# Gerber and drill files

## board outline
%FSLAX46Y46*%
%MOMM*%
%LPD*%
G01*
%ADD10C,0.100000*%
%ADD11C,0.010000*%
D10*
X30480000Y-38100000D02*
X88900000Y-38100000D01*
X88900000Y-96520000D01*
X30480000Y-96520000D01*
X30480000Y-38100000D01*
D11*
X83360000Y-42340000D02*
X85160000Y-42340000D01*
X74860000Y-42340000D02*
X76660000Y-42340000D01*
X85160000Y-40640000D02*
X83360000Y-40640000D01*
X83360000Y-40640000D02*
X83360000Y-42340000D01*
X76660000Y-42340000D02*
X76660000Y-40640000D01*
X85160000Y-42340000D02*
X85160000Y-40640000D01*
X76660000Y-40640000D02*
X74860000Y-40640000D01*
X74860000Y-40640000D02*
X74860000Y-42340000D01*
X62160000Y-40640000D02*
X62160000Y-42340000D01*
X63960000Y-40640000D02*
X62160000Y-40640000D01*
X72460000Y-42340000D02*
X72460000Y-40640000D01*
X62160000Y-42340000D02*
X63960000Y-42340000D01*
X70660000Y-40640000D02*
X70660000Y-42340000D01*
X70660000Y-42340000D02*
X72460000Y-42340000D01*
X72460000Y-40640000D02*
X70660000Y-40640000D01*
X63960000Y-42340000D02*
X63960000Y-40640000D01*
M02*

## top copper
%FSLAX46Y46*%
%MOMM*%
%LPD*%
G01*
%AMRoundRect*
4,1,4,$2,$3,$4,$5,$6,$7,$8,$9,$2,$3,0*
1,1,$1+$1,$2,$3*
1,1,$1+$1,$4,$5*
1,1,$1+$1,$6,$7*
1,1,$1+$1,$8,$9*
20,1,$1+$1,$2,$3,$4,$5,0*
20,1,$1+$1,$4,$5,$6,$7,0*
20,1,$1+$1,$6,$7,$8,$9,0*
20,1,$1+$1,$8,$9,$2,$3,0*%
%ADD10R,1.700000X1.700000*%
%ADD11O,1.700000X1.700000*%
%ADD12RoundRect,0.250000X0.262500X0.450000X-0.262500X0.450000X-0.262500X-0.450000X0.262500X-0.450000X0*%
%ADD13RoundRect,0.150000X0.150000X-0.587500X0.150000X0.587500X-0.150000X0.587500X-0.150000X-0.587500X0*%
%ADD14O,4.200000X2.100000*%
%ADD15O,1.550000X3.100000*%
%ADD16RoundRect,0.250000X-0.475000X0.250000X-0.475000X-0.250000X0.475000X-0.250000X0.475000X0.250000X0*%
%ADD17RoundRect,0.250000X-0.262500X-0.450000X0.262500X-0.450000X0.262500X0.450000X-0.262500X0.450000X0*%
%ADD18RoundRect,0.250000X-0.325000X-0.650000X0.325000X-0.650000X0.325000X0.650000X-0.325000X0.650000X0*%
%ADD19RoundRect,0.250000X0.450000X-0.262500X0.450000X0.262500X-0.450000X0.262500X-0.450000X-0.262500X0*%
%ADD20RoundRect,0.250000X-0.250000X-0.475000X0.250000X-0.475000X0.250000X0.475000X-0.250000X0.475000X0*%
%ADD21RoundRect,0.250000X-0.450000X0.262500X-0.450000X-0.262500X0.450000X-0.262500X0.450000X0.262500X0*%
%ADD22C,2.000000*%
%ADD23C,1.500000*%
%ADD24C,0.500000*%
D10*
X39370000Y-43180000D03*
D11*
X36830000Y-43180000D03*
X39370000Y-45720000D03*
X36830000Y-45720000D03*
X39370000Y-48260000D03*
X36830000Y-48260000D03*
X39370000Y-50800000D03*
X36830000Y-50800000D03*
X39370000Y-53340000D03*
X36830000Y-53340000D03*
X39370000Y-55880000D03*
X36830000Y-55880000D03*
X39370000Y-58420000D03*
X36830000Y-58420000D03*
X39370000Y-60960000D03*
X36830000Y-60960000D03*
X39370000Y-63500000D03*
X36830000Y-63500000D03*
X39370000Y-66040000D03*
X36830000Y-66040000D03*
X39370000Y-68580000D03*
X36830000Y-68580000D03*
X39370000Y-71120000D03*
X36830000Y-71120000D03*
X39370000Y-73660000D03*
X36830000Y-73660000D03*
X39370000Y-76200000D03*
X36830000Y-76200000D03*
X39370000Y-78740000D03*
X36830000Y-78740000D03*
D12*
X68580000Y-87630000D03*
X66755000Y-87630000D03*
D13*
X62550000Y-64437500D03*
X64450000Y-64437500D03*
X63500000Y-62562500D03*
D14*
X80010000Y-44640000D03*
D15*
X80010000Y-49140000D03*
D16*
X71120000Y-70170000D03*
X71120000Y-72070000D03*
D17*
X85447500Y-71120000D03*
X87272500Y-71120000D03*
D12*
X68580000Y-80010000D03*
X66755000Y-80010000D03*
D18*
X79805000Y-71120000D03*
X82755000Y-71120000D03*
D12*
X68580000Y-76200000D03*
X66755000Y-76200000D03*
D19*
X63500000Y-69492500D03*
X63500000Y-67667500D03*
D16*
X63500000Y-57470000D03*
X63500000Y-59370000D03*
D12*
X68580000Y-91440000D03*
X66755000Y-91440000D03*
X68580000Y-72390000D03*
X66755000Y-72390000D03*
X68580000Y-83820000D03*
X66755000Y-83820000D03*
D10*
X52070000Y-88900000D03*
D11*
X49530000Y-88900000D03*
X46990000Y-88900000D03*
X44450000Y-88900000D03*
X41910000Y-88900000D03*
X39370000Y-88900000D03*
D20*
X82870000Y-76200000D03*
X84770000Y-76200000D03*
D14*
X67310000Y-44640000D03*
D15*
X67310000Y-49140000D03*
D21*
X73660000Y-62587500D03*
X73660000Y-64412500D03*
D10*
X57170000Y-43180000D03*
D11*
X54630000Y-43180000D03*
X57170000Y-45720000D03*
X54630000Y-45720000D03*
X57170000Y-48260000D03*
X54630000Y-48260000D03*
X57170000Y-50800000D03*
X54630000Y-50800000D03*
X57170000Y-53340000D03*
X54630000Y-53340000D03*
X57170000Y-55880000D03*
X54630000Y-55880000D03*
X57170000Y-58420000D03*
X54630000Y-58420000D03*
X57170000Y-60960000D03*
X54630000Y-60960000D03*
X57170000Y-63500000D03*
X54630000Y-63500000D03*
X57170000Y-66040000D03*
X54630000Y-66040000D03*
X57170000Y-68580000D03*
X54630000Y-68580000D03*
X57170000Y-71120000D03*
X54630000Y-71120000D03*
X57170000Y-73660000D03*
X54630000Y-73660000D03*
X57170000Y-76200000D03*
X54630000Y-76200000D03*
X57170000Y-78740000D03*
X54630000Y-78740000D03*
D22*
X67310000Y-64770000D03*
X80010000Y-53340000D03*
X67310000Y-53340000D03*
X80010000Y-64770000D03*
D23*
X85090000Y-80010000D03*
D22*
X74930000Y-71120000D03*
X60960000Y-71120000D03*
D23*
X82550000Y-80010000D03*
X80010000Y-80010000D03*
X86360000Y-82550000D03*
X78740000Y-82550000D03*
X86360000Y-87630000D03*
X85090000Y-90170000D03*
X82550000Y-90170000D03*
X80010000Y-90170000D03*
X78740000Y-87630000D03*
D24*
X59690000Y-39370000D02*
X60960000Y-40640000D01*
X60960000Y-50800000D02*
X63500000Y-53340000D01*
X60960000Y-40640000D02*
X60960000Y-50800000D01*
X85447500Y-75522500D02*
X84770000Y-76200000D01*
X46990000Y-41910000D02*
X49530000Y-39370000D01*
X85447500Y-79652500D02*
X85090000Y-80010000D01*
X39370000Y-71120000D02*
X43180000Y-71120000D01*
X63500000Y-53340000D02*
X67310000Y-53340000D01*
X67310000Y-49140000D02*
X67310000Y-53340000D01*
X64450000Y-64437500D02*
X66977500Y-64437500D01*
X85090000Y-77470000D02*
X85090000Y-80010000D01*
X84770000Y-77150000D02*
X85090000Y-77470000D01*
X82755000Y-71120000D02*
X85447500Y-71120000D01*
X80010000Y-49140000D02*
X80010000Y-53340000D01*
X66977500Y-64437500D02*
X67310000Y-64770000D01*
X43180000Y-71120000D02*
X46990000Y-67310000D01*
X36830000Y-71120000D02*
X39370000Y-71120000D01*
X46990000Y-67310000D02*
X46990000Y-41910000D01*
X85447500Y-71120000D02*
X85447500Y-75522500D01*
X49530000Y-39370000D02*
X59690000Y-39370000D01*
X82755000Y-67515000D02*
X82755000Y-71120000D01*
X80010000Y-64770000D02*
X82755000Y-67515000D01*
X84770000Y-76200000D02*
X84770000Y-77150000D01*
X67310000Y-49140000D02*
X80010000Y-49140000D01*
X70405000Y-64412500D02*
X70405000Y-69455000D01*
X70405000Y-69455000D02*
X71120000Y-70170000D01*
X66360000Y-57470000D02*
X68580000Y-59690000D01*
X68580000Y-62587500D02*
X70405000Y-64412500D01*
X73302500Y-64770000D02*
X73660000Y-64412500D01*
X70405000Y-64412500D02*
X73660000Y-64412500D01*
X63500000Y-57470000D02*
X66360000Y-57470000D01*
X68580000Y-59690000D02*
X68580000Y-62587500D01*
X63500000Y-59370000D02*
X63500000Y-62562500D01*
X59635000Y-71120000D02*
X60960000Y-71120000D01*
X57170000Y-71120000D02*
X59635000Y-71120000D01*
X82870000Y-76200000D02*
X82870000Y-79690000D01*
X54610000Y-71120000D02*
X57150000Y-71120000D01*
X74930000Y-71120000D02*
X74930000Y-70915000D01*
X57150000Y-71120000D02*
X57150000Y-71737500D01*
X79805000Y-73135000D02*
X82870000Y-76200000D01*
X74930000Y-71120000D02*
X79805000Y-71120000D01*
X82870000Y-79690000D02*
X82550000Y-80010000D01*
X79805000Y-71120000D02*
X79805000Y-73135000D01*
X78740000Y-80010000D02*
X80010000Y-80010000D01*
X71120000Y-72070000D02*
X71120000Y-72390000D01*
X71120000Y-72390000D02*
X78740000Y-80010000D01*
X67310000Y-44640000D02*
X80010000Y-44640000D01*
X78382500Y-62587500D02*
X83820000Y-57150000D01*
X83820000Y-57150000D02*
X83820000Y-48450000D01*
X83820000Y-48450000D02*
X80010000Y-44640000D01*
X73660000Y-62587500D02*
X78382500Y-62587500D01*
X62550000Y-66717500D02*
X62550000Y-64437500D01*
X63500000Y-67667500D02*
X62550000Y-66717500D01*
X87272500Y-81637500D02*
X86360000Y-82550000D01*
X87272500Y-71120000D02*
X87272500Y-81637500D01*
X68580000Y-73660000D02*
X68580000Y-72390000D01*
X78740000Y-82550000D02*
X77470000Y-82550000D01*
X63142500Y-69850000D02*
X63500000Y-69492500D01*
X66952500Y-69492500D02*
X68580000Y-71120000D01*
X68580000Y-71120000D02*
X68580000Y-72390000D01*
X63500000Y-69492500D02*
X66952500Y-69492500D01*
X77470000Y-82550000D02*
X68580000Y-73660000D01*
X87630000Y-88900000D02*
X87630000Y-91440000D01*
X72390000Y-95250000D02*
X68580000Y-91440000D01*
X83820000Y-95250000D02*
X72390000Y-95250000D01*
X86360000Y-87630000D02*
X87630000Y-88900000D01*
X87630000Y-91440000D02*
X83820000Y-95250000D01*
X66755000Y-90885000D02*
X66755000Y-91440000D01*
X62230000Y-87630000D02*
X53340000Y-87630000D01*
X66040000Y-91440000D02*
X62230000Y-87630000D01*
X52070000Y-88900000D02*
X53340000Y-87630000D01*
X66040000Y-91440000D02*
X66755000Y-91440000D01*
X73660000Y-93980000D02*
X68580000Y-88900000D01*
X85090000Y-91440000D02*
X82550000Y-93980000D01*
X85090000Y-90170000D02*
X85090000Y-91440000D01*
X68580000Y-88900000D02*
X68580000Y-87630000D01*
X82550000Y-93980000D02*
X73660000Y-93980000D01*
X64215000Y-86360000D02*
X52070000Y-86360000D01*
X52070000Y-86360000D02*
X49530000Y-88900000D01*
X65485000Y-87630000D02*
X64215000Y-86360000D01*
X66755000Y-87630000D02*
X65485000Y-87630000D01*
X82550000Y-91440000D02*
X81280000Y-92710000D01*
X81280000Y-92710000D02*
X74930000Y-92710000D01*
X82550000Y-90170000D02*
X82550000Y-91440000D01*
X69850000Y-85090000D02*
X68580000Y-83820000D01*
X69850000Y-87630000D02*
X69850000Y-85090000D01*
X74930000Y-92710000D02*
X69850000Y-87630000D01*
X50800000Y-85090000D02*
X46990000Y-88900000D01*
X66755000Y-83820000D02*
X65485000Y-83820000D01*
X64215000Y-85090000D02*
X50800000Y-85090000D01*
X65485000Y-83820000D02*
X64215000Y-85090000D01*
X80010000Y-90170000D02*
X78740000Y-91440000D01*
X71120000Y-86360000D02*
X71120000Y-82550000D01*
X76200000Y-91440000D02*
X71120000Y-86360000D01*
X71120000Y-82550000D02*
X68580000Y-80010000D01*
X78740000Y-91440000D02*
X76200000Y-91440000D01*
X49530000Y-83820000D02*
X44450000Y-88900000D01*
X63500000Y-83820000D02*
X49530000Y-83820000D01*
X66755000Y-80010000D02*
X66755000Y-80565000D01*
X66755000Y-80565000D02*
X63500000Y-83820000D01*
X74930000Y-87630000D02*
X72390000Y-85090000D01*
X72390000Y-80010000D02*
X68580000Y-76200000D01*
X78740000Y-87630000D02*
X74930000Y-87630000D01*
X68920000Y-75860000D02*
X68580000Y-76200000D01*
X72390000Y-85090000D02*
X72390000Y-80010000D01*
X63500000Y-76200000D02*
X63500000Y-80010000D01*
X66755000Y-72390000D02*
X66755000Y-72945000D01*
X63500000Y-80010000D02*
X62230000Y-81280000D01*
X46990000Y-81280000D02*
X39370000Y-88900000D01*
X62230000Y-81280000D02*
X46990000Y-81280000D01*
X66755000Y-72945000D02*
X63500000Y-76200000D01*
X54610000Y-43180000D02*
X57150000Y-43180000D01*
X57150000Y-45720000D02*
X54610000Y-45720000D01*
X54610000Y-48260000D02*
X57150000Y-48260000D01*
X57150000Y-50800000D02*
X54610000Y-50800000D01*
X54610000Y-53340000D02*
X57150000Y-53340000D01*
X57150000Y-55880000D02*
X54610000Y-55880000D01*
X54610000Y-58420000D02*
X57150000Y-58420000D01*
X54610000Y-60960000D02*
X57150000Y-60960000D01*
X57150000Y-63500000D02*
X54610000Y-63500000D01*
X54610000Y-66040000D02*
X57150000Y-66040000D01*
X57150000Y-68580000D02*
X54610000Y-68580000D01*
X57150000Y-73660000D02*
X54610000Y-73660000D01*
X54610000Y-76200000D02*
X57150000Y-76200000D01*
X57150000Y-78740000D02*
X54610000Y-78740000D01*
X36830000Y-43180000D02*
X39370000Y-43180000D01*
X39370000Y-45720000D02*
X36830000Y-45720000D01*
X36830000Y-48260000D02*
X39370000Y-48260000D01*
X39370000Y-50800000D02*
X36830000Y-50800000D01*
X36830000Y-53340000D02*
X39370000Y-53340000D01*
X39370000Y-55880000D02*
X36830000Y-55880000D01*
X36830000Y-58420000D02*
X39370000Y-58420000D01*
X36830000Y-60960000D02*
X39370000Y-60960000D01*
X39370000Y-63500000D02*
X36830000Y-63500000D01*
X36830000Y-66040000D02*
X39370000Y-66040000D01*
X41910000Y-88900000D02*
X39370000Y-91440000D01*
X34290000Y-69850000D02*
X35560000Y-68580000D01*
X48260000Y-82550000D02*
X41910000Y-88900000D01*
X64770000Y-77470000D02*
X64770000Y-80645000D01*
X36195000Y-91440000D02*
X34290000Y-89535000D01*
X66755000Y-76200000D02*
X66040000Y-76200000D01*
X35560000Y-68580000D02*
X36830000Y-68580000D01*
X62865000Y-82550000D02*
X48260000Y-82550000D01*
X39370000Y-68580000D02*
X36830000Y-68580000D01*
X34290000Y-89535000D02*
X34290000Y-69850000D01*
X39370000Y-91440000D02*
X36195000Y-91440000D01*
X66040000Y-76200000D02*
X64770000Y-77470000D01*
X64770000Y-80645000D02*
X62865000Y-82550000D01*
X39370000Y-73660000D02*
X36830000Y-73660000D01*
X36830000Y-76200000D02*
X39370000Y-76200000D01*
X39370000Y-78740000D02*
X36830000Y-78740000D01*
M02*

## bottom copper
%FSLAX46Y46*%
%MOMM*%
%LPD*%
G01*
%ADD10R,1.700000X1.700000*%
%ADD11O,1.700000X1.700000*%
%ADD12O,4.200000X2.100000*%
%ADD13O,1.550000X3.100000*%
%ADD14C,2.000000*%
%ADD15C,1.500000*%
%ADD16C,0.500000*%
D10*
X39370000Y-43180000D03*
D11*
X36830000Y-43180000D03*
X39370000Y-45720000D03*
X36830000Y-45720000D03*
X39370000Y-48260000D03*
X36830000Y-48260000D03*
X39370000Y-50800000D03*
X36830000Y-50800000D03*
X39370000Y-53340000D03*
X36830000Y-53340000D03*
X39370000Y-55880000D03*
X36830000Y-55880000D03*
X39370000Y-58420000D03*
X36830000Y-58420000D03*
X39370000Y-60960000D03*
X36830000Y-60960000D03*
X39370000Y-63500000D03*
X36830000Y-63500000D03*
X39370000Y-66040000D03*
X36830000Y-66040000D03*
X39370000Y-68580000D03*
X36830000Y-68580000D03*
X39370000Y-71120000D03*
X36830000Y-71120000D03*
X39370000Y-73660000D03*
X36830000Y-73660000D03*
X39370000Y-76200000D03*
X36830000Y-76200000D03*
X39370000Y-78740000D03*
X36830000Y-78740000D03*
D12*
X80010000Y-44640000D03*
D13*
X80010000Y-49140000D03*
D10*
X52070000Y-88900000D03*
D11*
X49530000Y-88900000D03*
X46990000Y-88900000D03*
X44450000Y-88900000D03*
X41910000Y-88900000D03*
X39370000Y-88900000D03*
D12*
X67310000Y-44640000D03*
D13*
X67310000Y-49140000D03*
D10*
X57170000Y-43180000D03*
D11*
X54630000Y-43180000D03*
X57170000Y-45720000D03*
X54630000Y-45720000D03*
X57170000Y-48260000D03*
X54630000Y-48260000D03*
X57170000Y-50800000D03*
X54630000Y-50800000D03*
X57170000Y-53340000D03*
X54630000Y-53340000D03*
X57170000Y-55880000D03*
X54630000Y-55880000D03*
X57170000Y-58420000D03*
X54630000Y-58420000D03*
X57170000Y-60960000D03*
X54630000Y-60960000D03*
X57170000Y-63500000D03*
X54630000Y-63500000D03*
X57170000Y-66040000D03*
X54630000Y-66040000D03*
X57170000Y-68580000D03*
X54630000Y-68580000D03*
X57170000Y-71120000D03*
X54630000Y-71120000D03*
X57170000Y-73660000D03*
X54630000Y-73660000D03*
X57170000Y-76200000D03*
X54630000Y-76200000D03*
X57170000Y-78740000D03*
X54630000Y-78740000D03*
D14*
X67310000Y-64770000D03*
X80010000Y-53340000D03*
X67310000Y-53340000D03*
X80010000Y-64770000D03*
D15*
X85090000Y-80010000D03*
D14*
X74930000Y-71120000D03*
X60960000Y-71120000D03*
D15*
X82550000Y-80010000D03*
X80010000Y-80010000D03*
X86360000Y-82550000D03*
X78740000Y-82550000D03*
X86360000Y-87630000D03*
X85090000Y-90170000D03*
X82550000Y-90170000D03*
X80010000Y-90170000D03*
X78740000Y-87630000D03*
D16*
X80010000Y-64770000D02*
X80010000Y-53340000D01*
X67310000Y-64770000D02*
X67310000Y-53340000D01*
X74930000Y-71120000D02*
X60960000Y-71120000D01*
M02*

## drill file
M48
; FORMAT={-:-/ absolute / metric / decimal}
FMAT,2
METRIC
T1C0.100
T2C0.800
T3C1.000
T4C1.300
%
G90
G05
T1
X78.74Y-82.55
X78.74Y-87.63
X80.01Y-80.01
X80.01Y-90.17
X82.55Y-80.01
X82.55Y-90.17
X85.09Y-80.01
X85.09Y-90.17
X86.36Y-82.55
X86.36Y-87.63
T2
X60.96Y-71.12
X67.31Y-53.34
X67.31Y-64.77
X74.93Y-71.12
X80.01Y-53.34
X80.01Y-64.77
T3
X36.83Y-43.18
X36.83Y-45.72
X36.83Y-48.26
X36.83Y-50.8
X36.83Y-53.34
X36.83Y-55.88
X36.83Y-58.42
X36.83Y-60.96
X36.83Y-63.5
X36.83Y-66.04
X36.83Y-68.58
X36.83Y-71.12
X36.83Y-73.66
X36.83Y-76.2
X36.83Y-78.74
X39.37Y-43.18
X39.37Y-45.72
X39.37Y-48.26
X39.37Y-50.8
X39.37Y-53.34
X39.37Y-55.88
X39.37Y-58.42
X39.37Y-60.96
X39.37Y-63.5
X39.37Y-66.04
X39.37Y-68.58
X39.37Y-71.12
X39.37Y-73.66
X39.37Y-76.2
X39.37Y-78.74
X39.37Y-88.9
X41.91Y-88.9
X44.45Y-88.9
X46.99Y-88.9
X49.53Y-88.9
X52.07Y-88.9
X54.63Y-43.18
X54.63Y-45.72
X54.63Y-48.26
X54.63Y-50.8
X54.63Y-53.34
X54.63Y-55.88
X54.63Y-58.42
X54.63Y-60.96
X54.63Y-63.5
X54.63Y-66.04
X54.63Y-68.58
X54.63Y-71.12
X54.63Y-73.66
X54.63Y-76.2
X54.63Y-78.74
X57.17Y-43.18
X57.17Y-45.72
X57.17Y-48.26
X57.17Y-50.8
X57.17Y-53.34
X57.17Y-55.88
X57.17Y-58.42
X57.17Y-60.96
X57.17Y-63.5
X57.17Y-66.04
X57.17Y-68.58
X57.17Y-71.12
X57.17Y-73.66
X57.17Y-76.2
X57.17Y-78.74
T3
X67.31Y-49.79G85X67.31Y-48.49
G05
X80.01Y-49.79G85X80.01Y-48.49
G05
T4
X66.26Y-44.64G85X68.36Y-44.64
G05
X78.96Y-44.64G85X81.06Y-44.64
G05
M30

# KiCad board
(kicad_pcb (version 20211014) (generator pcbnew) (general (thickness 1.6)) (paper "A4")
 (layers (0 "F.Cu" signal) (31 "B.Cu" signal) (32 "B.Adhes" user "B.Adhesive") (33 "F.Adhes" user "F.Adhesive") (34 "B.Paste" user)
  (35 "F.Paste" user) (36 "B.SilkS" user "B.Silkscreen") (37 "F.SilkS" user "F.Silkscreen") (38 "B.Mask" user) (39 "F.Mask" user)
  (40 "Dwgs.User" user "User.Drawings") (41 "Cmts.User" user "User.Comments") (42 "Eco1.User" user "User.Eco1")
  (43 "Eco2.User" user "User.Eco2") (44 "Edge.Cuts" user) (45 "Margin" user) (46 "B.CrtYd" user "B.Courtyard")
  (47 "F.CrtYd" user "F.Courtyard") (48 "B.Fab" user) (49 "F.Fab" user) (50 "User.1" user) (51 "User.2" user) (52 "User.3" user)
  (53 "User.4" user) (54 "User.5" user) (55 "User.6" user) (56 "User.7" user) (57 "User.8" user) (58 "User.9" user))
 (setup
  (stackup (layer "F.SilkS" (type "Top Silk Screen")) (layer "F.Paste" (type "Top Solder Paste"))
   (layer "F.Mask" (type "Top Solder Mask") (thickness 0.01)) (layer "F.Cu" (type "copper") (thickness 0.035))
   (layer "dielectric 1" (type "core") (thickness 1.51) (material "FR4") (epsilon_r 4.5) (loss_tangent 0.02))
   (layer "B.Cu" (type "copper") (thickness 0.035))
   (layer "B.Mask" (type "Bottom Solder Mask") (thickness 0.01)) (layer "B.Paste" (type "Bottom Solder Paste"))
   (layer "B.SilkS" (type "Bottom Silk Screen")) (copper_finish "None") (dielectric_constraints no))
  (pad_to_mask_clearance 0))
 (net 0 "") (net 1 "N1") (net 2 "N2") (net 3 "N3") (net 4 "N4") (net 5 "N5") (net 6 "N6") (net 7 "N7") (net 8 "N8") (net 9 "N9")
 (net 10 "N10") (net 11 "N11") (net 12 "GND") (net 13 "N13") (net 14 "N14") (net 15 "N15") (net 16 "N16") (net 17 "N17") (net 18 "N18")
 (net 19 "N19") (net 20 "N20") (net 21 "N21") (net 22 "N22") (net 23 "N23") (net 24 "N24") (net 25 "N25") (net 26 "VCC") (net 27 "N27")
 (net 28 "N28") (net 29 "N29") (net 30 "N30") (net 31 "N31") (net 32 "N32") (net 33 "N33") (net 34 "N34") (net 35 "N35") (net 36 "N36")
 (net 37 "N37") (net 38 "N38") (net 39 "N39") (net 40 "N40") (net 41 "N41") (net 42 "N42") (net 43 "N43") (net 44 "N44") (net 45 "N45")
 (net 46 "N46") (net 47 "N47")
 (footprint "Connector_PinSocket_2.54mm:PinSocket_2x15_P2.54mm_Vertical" (layer "F.Cu") (at 39.37 43.18)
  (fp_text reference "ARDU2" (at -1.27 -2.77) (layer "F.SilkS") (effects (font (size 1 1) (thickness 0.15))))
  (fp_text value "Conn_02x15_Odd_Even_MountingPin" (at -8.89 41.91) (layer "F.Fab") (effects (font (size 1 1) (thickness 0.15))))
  (pad "1" thru_hole rect (at 0 0) (size 1.7 1.7) (drill 1) (layers *.Cu *.Mask) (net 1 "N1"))
  (pad "2" thru_hole oval (at -2.54 0) (size 1.7 1.7) (drill 1) (layers *.Cu *.Mask) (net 1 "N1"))
  (pad "3" thru_hole oval (at 0 2.54) (size 1.7 1.7) (drill 1) (layers *.Cu *.Mask) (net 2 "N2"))
  (pad "4" thru_hole oval (at -2.54 2.54) (size 1.7 1.7) (drill 1) (layers *.Cu *.Mask) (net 2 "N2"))
  (pad "5" thru_hole oval (at 0 5.08) (size 1.7 1.7) (drill 1) (layers *.Cu *.Mask) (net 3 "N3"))
  (pad "6" thru_hole oval (at -2.54 5.08) (size 1.7 1.7) (drill 1) (layers *.Cu *.Mask) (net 3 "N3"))
  (pad "7" thru_hole oval (at 0 7.62) (size 1.7 1.7) (drill 1) (layers *.Cu *.Mask) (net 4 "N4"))
  (pad "8" thru_hole oval (at -2.54 7.62) (size 1.7 1.7) (drill 1) (layers *.Cu *.Mask) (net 4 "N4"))
  (pad "9" thru_hole oval (at 0 10.16) (size 1.7 1.7) (drill 1) (layers *.Cu *.Mask) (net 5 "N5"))
  (pad "10" thru_hole oval (at -2.54 10.16) (size 1.7 1.7) (drill 1) (layers *.Cu *.Mask) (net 5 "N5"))
  (pad "11" thru_hole oval (at 0 12.7) (size 1.7 1.7) (drill 1) (layers *.Cu *.Mask) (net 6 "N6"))
  (pad "12" thru_hole oval (at -2.54 12.7) (size 1.7 1.7) (drill 1) (layers *.Cu *.Mask) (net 6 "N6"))
  (pad "13" thru_hole oval (at 0 15.24) (size 1.7 1.7) (drill 1) (layers *.Cu *.Mask) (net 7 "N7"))
  (pad "14" thru_hole oval (at -2.54 15.24) (size 1.7 1.7) (drill 1) (layers *.Cu *.Mask) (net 7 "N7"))
  (pad "15" thru_hole oval (at 0 17.78) (size 1.7 1.7) (drill 1) (layers *.Cu *.Mask) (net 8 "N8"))
  (pad "16" thru_hole oval (at -2.54 17.78) (size 1.7 1.7) (drill 1) (layers *.Cu *.Mask) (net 8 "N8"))
  (pad "17" thru_hole oval (at 0 20.32) (size 1.7 1.7) (drill 1) (layers *.Cu *.Mask) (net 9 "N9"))
  (pad "18" thru_hole oval (at -2.54 20.32) (size 1.7 1.7) (drill 1) (layers *.Cu *.Mask) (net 9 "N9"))
  (pad "19" thru_hole oval (at 0 22.86) (size 1.7 1.7) (drill 1) (layers *.Cu *.Mask) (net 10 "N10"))
  (pad "20" thru_hole oval (at -2.54 22.86) (size 1.7 1.7) (drill 1) (layers *.Cu *.Mask) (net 10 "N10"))
  (pad "21" thru_hole oval (at 0 25.4) (size 1.7 1.7) (drill 1) (layers *.Cu *.Mask) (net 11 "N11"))
  (pad "22" thru_hole oval (at -2.54 25.4) (size 1.7 1.7) (drill 1) (layers *.Cu *.Mask) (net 11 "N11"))
  (pad "23" thru_hole oval (at 0 27.94) (size 1.7 1.7) (drill 1) (layers *.Cu *.Mask) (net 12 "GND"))
  (pad "24" thru_hole oval (at -2.54 27.94) (size 1.7 1.7) (drill 1) (layers *.Cu *.Mask) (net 12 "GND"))
  (pad "25" thru_hole oval (at 0 30.48) (size 1.7 1.7) (drill 1) (layers *.Cu *.Mask) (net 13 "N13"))
  (pad "26" thru_hole oval (at -2.54 30.48) (size 1.7 1.7) (drill 1) (layers *.Cu *.Mask) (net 13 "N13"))
  (pad "27" thru_hole oval (at 0 33.02) (size 1.7 1.7) (drill 1) (layers *.Cu *.Mask) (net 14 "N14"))
  (pad "28" thru_hole oval (at -2.54 33.02) (size 1.7 1.7) (drill 1) (layers *.Cu *.Mask) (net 14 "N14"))
  (pad "29" thru_hole oval (at 0 35.56) (size 1.7 1.7) (drill 1) (layers *.Cu *.Mask) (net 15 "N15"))
  (pad "30" thru_hole oval (at -2.54 35.56) (size 1.7 1.7) (drill 1) (layers *.Cu *.Mask) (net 15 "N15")))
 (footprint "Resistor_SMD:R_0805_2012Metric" (layer "F.Cu") (at 67.6675 87.63 180)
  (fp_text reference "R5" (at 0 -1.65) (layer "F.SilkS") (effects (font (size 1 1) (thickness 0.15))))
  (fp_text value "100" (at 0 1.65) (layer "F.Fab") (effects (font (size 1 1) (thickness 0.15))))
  (pad "1" smd roundrect (at -0.9125 0 180) (size 1.025 1.4) (layers "F.Cu" "F.Paste" "F.Mask") (roundrect_rratio 0.243902439)
   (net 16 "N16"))
  (pad "2" smd roundrect (at 0.9125 0 180) (size 1.025 1.4) (layers "F.Cu" "F.Paste" "F.Mask") (roundrect_rratio 0.243902439) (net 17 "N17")))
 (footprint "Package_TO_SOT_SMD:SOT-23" (layer "F.Cu") (at 63.5 63.5 90)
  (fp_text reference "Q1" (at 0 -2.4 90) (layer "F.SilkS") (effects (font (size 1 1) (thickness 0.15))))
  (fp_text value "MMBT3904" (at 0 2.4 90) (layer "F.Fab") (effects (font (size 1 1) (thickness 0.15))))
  (pad "1" smd roundrect (at -0.9375 -0.95 90) (size 1.475 0.6) (layers "F.Cu" "F.Paste" "F.Mask") (roundrect_rratio 0.25) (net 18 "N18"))
  (pad "2" smd roundrect (at -0.9375 0.95 90) (size 1.475 0.6) (layers "F.Cu" "F.Paste" "F.Mask") (roundrect_rratio 0.25) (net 12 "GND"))
  (pad "3" smd roundrect (at 0.9375 0 90) (size 1.475 0.6) (layers "F.Cu" "F.Paste" "F.Mask") (roundrect_rratio 0.25) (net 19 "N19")))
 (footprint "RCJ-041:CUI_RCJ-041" (layer "F.Cu") (at 80.01 40.64 90)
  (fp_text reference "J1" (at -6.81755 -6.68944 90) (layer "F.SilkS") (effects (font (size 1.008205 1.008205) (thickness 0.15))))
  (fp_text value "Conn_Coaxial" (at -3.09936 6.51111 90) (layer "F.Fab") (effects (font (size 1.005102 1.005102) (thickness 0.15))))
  (fp_line (start -1.7 3.35) (end -1.7 5.15) (layer "Edge.Cuts") (width 0.01))
  (fp_line (start -1.7 -5.15) (end -1.7 -3.35) (layer "Edge.Cuts") (width 0.01))
  (fp_line (start 0 5.15) (end 0 3.35) (layer "Edge.Cuts") (width 0.01))
  (fp_line (start 0 3.35) (end -1.7 3.35) (layer "Edge.Cuts") (width 0.01))
  (fp_line (start -1.7 -3.35) (end 0 -3.35) (layer "Edge.Cuts") (width 0.01))
  (fp_line (start -1.7 5.15) (end 0 5.15) (layer "Edge.Cuts") (width 0.01))
  (fp_line (start 0 -3.35) (end 0 -5.15) (layer "Edge.Cuts") (width 0.01))
  (fp_line (start 0 -5.15) (end -1.7 -5.15) (layer "Edge.Cuts") (width 0.01))
  (pad "1" thru_hole oval locked (at -4 0 90) (size 2.1 4.2) (drill oval 1.3 3.4) (layers *.Cu *.Mask) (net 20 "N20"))
  (pad "2" thru_hole oval locked (at -8.5 0 90) (size 3.1 1.55) (drill oval 2.3 1) (layers *.Cu *.Mask) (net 12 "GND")))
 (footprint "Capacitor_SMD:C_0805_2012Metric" (layer "F.Cu") (at 71.12 71.12 -90)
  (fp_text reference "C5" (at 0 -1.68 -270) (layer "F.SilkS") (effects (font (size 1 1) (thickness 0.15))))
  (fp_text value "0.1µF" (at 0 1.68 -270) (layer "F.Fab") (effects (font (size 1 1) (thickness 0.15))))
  (pad "1" smd roundrect (at -0.95 0 270) (size 1 1.45) (layers "F.Cu" "F.Paste" "F.Mask") (roundrect_rratio 0.25) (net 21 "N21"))
  (pad "2" smd roundrect (at 0.95 0 270) (size 1 1.45) (layers "F.Cu" "F.Paste" "F.Mask") (roundrect_rratio 0.25) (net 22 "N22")))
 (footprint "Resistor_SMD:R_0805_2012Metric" (layer "F.Cu") (at 86.36 71.12)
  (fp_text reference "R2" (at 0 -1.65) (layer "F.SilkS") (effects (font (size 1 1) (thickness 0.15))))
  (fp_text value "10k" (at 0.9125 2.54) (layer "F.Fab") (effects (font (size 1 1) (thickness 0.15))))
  (pad "1" smd roundrect (at -0.9125 0) (size 1.025 1.4) (layers "F.Cu" "F.Paste" "F.Mask") (roundrect_rratio 0.243902439) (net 12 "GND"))
  (pad "2" smd roundrect (at 0.9125 0) (size 1.025 1.4) (layers "F.Cu" "F.Paste" "F.Mask") (roundrect_rratio 0.243902439) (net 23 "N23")))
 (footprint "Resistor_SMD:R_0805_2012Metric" (layer "F.Cu") (at 67.6675 80.01 180)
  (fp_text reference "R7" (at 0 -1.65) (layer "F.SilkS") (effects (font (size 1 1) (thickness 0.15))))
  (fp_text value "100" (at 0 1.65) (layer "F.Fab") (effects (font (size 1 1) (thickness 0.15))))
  (pad "1" smd roundrect (at -0.9125 0 180) (size 1.025 1.4) (layers "F.Cu" "F.Paste" "F.Mask") (roundrect_rratio 0.243902439)
   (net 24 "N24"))
  (pad "2" smd roundrect (at 0.9125 0 180) (size 1.025 1.4) (layers "F.Cu" "F.Paste" "F.Mask") (roundrect_rratio 0.243902439) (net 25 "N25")))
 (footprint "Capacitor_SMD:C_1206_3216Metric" (layer "F.Cu") (at 81.28 71.12)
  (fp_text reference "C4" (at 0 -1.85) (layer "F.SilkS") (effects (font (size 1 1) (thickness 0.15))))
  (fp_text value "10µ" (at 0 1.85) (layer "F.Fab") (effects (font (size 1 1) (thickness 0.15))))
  (pad "1" smd roundrect (at -1.475 0) (size 1.15 1.8) (layers "F.Cu" "F.Paste" "F.Mask") (roundrect_rratio 0.2173913043) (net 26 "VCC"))
  (pad "2" smd roundrect (at 1.475 0) (size 1.15 1.8) (layers "F.Cu" "F.Paste" "F.Mask") (roundrect_rratio 0.2173913043) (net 12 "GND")))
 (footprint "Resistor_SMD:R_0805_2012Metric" (layer "F.Cu") (at 67.6675 76.2 180)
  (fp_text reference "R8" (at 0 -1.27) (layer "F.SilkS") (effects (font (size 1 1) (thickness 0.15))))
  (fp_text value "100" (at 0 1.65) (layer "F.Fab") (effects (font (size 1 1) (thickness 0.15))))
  (pad "1" smd roundrect (at -0.9125 0 180) (size 1.025 1.4) (layers "F.Cu" "F.Paste" "F.Mask") (roundrect_rratio 0.243902439)
   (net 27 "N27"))
  (pad "2" smd roundrect (at 0.9125 0 180) (size 1.025 1.4) (layers "F.Cu" "F.Paste" "F.Mask") (roundrect_rratio 0.243902439) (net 11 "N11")))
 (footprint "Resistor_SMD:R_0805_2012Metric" (layer "F.Cu") (at 63.5 68.58 90)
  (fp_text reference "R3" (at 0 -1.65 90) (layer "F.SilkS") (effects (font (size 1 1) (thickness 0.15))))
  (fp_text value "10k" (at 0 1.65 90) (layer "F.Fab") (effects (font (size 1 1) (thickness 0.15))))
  (pad "1" smd roundrect (at -0.9125 0 90) (size 1.025 1.4) (layers "F.Cu" "F.Paste" "F.Mask") (roundrect_rratio 0.243902439) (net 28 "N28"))
  (pad "2" smd roundrect (at 0.9125 0 90) (size 1.025 1.4) (layers "F.Cu" "F.Paste" "F.Mask") (roundrect_rratio 0.243902439) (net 18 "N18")))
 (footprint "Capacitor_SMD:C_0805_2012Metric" (layer "F.Cu") (at 63.5 58.42 -90)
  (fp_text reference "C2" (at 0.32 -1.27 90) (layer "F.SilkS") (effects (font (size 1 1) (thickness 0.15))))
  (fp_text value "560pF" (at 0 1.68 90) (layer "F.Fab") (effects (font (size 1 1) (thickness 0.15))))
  (pad "1" smd roundrect (at -0.95 0 270) (size 1 1.45) (layers "F.Cu" "F.Paste" "F.Mask") (roundrect_rratio 0.25) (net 21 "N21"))
  (pad "2" smd roundrect (at 0.95 0 270) (size 1 1.45) (layers "F.Cu" "F.Paste" "F.Mask") (roundrect_rratio 0.25) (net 19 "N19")))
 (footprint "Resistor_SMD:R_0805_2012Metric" (layer "F.Cu") (at 67.6675 91.44 180)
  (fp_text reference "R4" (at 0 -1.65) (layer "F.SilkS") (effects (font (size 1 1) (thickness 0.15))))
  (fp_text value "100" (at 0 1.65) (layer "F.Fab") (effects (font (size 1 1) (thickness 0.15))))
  (pad "1" smd roundrect (at -0.9125 0 180) (size 1.025 1.4) (layers "F.Cu" "F.Paste" "F.Mask") (roundrect_rratio 0.243902439)
   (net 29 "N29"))
  (pad "2" smd roundrect (at 0.9125 0 180) (size 1.025 1.4) (layers "F.Cu" "F.Paste" "F.Mask") (roundrect_rratio 0.243902439) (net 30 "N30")))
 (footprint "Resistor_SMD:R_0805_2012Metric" (layer "F.Cu") (at 67.6675 72.39 180)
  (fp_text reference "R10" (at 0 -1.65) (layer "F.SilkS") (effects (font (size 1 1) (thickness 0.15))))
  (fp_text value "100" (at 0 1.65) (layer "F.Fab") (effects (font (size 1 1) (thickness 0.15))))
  (pad "1" smd roundrect (at -0.9125 0 180) (size 1.025 1.4) (layers "F.Cu" "F.Paste" "F.Mask") (roundrect_rratio 0.243902439)
   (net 28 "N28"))
  (pad "2" smd roundrect (at 0.9125 0 180) (size 1.025 1.4) (layers "F.Cu" "F.Paste" "F.Mask") (roundrect_rratio 0.243902439) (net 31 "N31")))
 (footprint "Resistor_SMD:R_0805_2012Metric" (layer "F.Cu") (at 67.6675 83.82 180)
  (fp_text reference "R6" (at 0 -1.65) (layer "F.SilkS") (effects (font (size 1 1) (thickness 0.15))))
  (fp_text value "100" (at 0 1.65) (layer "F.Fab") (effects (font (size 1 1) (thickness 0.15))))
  (pad "1" smd roundrect (at -0.9125 0 180) (size 1.025 1.4) (layers "F.Cu" "F.Paste" "F.Mask") (roundrect_rratio 0.243902439)
   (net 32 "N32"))
  (pad "2" smd roundrect (at 0.9125 0 180) (size 1.025 1.4) (layers "F.Cu" "F.Paste" "F.Mask") (roundrect_rratio 0.243902439) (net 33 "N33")))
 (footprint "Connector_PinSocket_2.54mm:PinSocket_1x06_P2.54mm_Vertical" (layer "F.Cu") (at 52.07 88.9 -90)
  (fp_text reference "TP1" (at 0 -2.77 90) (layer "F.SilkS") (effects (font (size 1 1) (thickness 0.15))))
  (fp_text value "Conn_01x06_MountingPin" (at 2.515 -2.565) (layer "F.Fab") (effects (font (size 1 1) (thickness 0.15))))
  (pad "1" thru_hole rect (at 0 0 270) (size 1.7 1.7) (drill 1) (layers *.Cu *.Mask) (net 30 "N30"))
  (pad "2" thru_hole oval (at 0 2.54 270) (size 1.7 1.7) (drill 1) (layers *.Cu *.Mask) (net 17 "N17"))
  (pad "3" thru_hole oval (at 0 5.08 270) (size 1.7 1.7) (drill 1) (layers *.Cu *.Mask) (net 33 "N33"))
  (pad "4" thru_hole oval (at 0 7.62 270) (size 1.7 1.7) (drill 1) (layers *.Cu *.Mask) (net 25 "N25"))
  (pad "5" thru_hole oval (at 0 10.16 270) (size 1.7 1.7) (drill 1) (layers *.Cu *.Mask) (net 11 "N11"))
  (pad "6" thru_hole oval (at 0 12.7 270) (size 1.7 1.7) (drill 1) (layers *.Cu *.Mask) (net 31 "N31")))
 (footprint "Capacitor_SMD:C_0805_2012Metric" (layer "F.Cu") (at 83.82 76.2)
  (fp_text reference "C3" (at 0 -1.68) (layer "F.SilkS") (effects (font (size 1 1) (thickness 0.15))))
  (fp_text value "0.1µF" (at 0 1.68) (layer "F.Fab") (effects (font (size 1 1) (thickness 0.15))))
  (pad "1" smd roundrect (at -0.95 0) (size 1 1.45) (layers "F.Cu" "F.Paste" "F.Mask") (roundrect_rratio 0.25) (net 26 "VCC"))
  (pad "2" smd roundrect (at 0.95 0) (size 1 1.45) (layers "F.Cu" "F.Paste" "F.Mask") (roundrect_rratio 0.25) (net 12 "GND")))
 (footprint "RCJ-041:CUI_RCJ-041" (layer "F.Cu") (at 67.31 40.64 90)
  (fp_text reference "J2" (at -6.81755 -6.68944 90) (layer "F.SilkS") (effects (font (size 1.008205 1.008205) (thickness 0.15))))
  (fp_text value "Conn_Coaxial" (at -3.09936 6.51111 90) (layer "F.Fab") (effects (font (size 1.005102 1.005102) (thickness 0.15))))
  (fp_line (start 0 -5.15) (end -1.7 -5.15) (layer "Edge.Cuts") (width 0.01))
  (fp_line (start 0 -3.35) (end 0 -5.15) (layer "Edge.Cuts") (width 0.01))
  (fp_line (start -1.7 5.15) (end 0 5.15) (layer "Edge.Cuts") (width 0.01))
  (fp_line (start -1.7 -5.15) (end -1.7 -3.35) (layer "Edge.Cuts") (width 0.01))
  (fp_line (start 0 3.35) (end -1.7 3.35) (layer "Edge.Cuts") (width 0.01))
  (fp_line (start -1.7 3.35) (end -1.7 5.15) (layer "Edge.Cuts") (width 0.01))
  (fp_line (start 0 5.15) (end 0 3.35) (layer "Edge.Cuts") (width 0.01))
  (fp_line (start -1.7 -3.35) (end 0 -3.35) (layer "Edge.Cuts") (width 0.01))
  (pad "1" thru_hole oval locked (at -4 0 90) (size 2.1 4.2) (drill oval 1.3 3.4) (layers *.Cu *.Mask) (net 20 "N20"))
  (pad "2" thru_hole oval locked (at -8.5 0 90) (size 3.1 1.55) (drill oval 2.3 1) (layers *.Cu *.Mask) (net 12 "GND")))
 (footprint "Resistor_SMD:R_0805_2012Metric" (layer "F.Cu") (at 73.66 63.5 -90)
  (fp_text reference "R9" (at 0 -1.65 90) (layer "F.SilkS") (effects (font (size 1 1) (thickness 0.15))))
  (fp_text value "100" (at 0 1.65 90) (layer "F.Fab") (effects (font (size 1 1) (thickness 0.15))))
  (pad "1" smd roundrect (at -0.9125 0 270) (size 1.025 1.4) (layers "F.Cu" "F.Paste" "F.Mask") (roundrect_rratio 0.243902439)
   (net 20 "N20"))
  (pad "2" smd roundrect (at 0.9125 0 270) (size 1.025 1.4) (layers "F.Cu" "F.Paste" "F.Mask") (roundrect_rratio 0.243902439) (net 21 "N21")))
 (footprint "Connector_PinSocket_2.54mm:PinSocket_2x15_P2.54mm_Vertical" (layer "F.Cu") (at 57.17 43.18)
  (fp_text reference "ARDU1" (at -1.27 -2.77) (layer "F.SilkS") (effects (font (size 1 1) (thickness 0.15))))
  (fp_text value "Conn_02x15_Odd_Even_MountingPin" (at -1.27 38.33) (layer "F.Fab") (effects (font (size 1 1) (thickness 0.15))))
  (pad "1" thru_hole rect (at 0 0) (size 1.7 1.7) (drill 1) (layers *.Cu *.Mask) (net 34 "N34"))
  (pad "2" thru_hole oval (at -2.54 0) (size 1.7 1.7) (drill 1) (layers *.Cu *.Mask) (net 34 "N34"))
  (pad "3" thru_hole oval (at 0 2.54) (size 1.7 1.7) (drill 1) (layers *.Cu *.Mask) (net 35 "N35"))
  (pad "4" thru_hole oval (at -2.54 2.54) (size 1.7 1.7) (drill 1) (layers *.Cu *.Mask) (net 35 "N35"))
  (pad "5" thru_hole oval (at 0 5.08) (size 1.7 1.7) (drill 1) (layers *.Cu *.Mask) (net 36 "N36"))
  (pad "6" thru_hole oval (at -2.54 5.08) (size 1.7 1.7) (drill 1) (layers *.Cu *.Mask) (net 36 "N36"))
  (pad "7" thru_hole oval (at 0 7.62) (size 1.7 1.7) (drill 1) (layers *.Cu *.Mask) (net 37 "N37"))
  (pad "8" thru_hole oval (at -2.54 7.62) (size 1.7 1.7) (drill 1) (layers *.Cu *.Mask) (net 37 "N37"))
  (pad "9" thru_hole oval (at 0 10.16) (size 1.7 1.7) (drill 1) (layers *.Cu *.Mask) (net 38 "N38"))
  (pad "10" thru_hole oval (at -2.54 10.16) (size 1.7 1.7) (drill 1) (layers *.Cu *.Mask) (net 38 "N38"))
  (pad "11" thru_hole oval (at 0 12.7) (size 1.7 1.7) (drill 1) (layers *.Cu *.Mask) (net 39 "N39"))
  (pad "12" thru_hole oval (at -2.54 12.7) (size 1.7 1.7) (drill 1) (layers *.Cu *.Mask) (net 39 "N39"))
  (pad "13" thru_hole oval (at 0 15.24) (size 1.7 1.7) (drill 1) (layers *.Cu *.Mask) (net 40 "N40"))
  (pad "14" thru_hole oval (at -2.54 15.24) (size 1.7 1.7) (drill 1) (layers *.Cu *.Mask) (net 40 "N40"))
  (pad "15" thru_hole oval (at 0 17.78) (size 1.7 1.7) (drill 1) (layers *.Cu *.Mask) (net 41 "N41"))
  (pad "16" thru_hole oval (at -2.54 17.78) (size 1.7 1.7) (drill 1) (layers *.Cu *.Mask) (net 41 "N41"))
  (pad "17" thru_hole oval (at 0 20.32) (size 1.7 1.7) (drill 1) (layers *.Cu *.Mask) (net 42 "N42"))
  (pad "18" thru_hole oval (at -2.54 20.32) (size 1.7 1.7) (drill 1) (layers *.Cu *.Mask) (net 42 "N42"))
  (pad "19" thru_hole oval (at 0 22.86) (size 1.7 1.7) (drill 1) (layers *.Cu *.Mask) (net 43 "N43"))
  (pad "20" thru_hole oval (at -2.54 22.86) (size 1.7 1.7) (drill 1) (layers *.Cu *.Mask) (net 43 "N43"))
  (pad "21" thru_hole oval (at 0 25.4) (size 1.7 1.7) (drill 1) (layers *.Cu *.Mask) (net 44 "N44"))
  (pad "22" thru_hole oval (at -2.54 25.4) (size 1.7 1.7) (drill 1) (layers *.Cu *.Mask) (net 44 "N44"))
  (pad "23" thru_hole oval (at 0 27.94) (size 1.7 1.7) (drill 1) (layers *.Cu *.Mask) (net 26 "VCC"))
  (pad "24" thru_hole oval (at -2.54 27.94) (size 1.7 1.7) (drill 1) (layers *.Cu *.Mask) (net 26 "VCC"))
  (pad "25" thru_hole oval (at 0 30.48) (size 1.7 1.7) (drill 1) (layers *.Cu *.Mask) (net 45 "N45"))
  (pad "26" thru_hole oval (at -2.54 30.48) (size 1.7 1.7) (drill 1) (layers *.Cu *.Mask) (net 45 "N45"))
  (pad "27" thru_hole oval (at 0 33.02) (size 1.7 1.7) (drill 1) (layers *.Cu *.Mask) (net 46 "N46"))
  (pad "28" thru_hole oval (at -2.54 33.02) (size 1.7 1.7) (drill 1) (layers *.Cu *.Mask) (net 46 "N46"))
  (pad "29" thru_hole oval (at 0 35.56) (size 1.7 1.7) (drill 1) (layers *.Cu *.Mask) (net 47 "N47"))
  (pad "30" thru_hole oval (at -2.54 35.56) (size 1.7 1.7) (drill 1) (layers *.Cu *.Mask) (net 47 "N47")))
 (gr_rect (start 88.9 38.1) (end 30.48 96.52) (layer "Edge.Cuts") (width 0.1) (fill none))
 (segment (start 59.69 39.37) (end 60.96 40.64) (width 0.5) (layer "F.Cu") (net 12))
 (segment (start 60.96 50.8) (end 63.5 53.34) (width 0.5) (layer "F.Cu") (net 12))
 (segment (start 60.96 40.64) (end 60.96 50.8) (width 0.5) (layer "F.Cu") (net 12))
 (segment (start 85.4475 75.5225) (end 84.77 76.2) (width 0.5) (layer "F.Cu") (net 12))
 (segment (start 46.99 41.91) (end 49.53 39.37) (width 0.5) (layer "F.Cu") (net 12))
 (segment (start 85.4475 79.6525) (end 85.09 80.01) (width 0.5) (layer "F.Cu") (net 12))
 (segment (start 39.37 71.12) (end 43.18 71.12) (width 0.5) (layer "F.Cu") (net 12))
 (segment (start 63.5 53.34) (end 67.31 53.34) (width 0.5) (layer "F.Cu") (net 12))
 (segment (start 67.31 49.14) (end 67.31 53.34) (width 0.5) (layer "F.Cu") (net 12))
 (segment (start 64.45 64.4375) (end 66.9775 64.4375) (width 0.5) (layer "F.Cu") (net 12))
 (segment (start 85.09 77.47) (end 85.09 80.01) (width 0.5) (layer "F.Cu") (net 12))
 (segment (start 84.77 77.15) (end 85.09 77.47) (width 0.5) (layer "F.Cu") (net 12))
 (segment (start 82.755 71.12) (end 85.4475 71.12) (width 0.5) (layer "F.Cu") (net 12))
 (segment (start 80.01 49.14) (end 80.01 53.34) (width 0.5) (layer "F.Cu") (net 12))
 (segment (start 66.9775 64.4375) (end 67.31 64.77) (width 0.5) (layer "F.Cu") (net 12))
 (segment (start 43.18 71.12) (end 46.99 67.31) (width 0.5) (layer "F.Cu") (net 12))
 (segment (start 36.83 71.12) (end 39.37 71.12) (width 0.5) (layer "F.Cu") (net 12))
 (segment (start 46.99 67.31) (end 46.99 41.91) (width 0.5) (layer "F.Cu") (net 12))
 (segment (start 85.4475 71.12) (end 85.4475 75.5225) (width 0.5) (layer "F.Cu") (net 12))
 (segment (start 49.53 39.37) (end 59.69 39.37) (width 0.5) (layer "F.Cu") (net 12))
 (segment (start 82.755 67.515) (end 82.755 71.12) (width 0.5) (layer "F.Cu") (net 12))
 (segment (start 80.01 64.77) (end 82.755 67.515) (width 0.5) (layer "F.Cu") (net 12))
 (segment (start 84.77 76.2) (end 84.77 77.15) (width 0.5) (layer "F.Cu") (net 12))
 (segment (start 67.31 49.14) (end 80.01 49.14) (width 0.5) (layer "F.Cu") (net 12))
 (via (at 67.31 64.77) (size 2) (drill 0.8) (layers "F.Cu" "B.Cu") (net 12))
 (via (at 80.01 53.34) (size 2) (drill 0.8) (layers "F.Cu" "B.Cu") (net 12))
 (via (at 67.31 53.34) (size 2) (drill 0.8) (layers "F.Cu" "B.Cu") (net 12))
 (via (at 80.01 64.77) (size 2) (drill 0.8) (layers "F.Cu" "B.Cu") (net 12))
 (via (at 85.09 80.01) (size 1.5) (drill 0.1) (layers "F.Cu" "B.Cu") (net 12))
 (segment (start 80.01 64.77) (end 80.01 53.34) (width 0.5) (layer "B.Cu") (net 12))
 (segment (start 67.31 64.77) (end 67.31 53.34) (width 0.5) (layer "B.Cu") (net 12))
 (segment (start 70.405 64.4125) (end 70.405 69.455) (width 0.5) (layer "F.Cu") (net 21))
 (segment (start 70.405 69.455) (end 71.12 70.17) (width 0.5) (layer "F.Cu") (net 21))
 (segment (start 66.36 57.47) (end 68.58 59.69) (width 0.5) (layer "F.Cu") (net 21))
 (segment (start 68.58 62.5875) (end 70.405 64.4125) (width 0.5) (layer "F.Cu") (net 21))
 (segment (start 73.3025 64.77) (end 73.66 64.4125) (width 0.5) (layer "F.Cu") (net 21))
 (segment (start 70.405 64.4125) (end 73.66 64.4125) (width 0.5) (layer "F.Cu") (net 21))
 (segment (start 63.5 57.47) (end 66.36 57.47) (width 0.5) (layer "F.Cu") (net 21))
 (segment (start 68.58 59.69) (end 68.58 62.5875) (width 0.5) (layer "F.Cu") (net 21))
 (segment (start 63.5 59.37) (end 63.5 62.5625) (width 0.5) (layer "F.Cu") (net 19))
 (segment (start 59.635 71.12) (end 60.96 71.12) (width 0.5) (layer "F.Cu") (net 26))
 (segment (start 57.17 71.12) (end 59.635 71.12) (width 0.5) (layer "F.Cu") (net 26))
 (segment (start 82.87 76.2) (end 82.87 79.69) (width 0.5) (layer "F.Cu") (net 26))
 (segment (start 54.61 71.12) (end 57.15 71.12) (width 0.5) (layer "F.Cu") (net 26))
 (segment (start 74.93 71.12) (end 74.93 70.915) (width 0.5) (layer "F.Cu") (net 26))
 (segment (start 57.15 71.12) (end 57.15 71.7375) (width 0.5) (layer "F.Cu") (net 26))
 (segment (start 79.805 73.135) (end 82.87 76.2) (width 0.5) (layer "F.Cu") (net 26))
 (segment (start 74.93 71.12) (end 79.805 71.12) (width 0.5) (layer "F.Cu") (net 26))
 (segment (start 82.87 79.69) (end 82.55 80.01) (width 0.5) (layer "F.Cu") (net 26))
 (segment (start 79.805 71.12) (end 79.805 73.135) (width 0.5) (layer "F.Cu") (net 26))
 (via (at 74.93 71.12) (size 2) (drill 0.8) (layers "F.Cu" "B.Cu") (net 26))
 (via (at 60.96 71.12) (size 2) (drill 0.8) (layers "F.Cu" "B.Cu") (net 26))
 (via (at 82.55 80.01) (size 1.5) (drill 0.1) (layers "F.Cu" "B.Cu") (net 26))
 (segment (start 74.93 71.12) (end 60.96 71.12) (width 0.5) (layer "B.Cu") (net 26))
 (segment (start 78.74 80.01) (end 80.01 80.01) (width 0.5) (layer "F.Cu") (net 22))
 (segment (start 71.12 72.07) (end 71.12 72.39) (width 0.5) (layer "F.Cu") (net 22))
 (segment (start 71.12 72.39) (end 78.74 80.01) (width 0.5) (layer "F.Cu") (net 22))
 (via (at 80.01 80.01) (size 1.5) (drill 0.1) (layers "F.Cu" "B.Cu") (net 22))
 (segment (start 67.31 44.64) (end 80.01 44.64) (width 0.5) (layer "F.Cu") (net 20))
 (segment (start 78.3825 62.5875) (end 83.82 57.15) (width 0.5) (layer "F.Cu") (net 20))
 (segment (start 83.82 57.15) (end 83.82 48.45) (width 0.5) (layer "F.Cu") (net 20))
 (segment (start 83.82 48.45) (end 80.01 44.64) (width 0.5) (layer "F.Cu") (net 20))
 (segment (start 73.66 62.5875) (end 78.3825 62.5875) (width 0.5) (layer "F.Cu") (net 20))
 (segment (start 62.55 66.7175) (end 62.55 64.4375) (width 0.5) (layer "F.Cu") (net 18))
 (segment (start 63.5 67.6675) (end 62.55 66.7175) (width 0.5) (layer "F.Cu") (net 18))
 (segment (start 87.2725 81.6375) (end 86.36 82.55) (width 0.5) (layer "F.Cu") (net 23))
 (segment (start 87.2725 71.12) (end 87.2725 81.6375) (width 0.5) (layer "F.Cu") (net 23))
 (via (at 86.36 82.55) (size 1.5) (drill 0.1) (layers "F.Cu" "B.Cu") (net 23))
 (segment (start 68.58 73.66) (end 68.58 72.39) (width 0.5) (layer "F.Cu") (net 28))
 (segment (start 78.74 82.55) (end 77.47 82.55) (width 0.5) (layer "F.Cu") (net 28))
 (segment (start 63.1425 69.85) (end 63.5 69.4925) (width 0.5) (layer "F.Cu") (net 28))
 (segment (start 66.9525 69.4925) (end 68.58 71.12) (width 0.5) (layer "F.Cu") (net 28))
 (segment (start 68.58 71.12) (end 68.58 72.39) (width 0.5) (layer "F.Cu") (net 28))
 (segment (start 63.5 69.4925) (end 66.9525 69.4925) (width 0.5) (layer "F.Cu") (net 28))
 (segment (start 77.47 82.55) (end 68.58 73.66) (width 0.5) (layer "F.Cu") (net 28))
 (via (at 78.74 82.55) (size 1.5) (drill 0.1) (layers "F.Cu" "B.Cu") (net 28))
 (segment (start 87.63 88.9) (end 87.63 91.44) (width 0.5) (layer "F.Cu") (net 29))
 (segment (start 72.39 95.25) (end 68.58 91.44) (width 0.5) (layer "F.Cu") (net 29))
 (segment (start 83.82 95.25) (end 72.39 95.25) (width 0.5) (layer "F.Cu") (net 29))
 (segment (start 86.36 87.63) (end 87.63 88.9) (width 0.5) (layer "F.Cu") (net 29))
 (segment (start 87.63 91.44) (end 83.82 95.25) (width 0.5) (layer "F.Cu") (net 29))
 (via (at 86.36 87.63) (size 1.5) (drill 0.1) (layers "F.Cu" "B.Cu") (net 29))
 (segment (start 66.755 90.885) (end 66.755 91.44) (width 0.5) (layer "F.Cu") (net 30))
 (segment (start 62.23 87.63) (end 53.34 87.63) (width 0.5) (layer "F.Cu") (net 30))
 (segment (start 66.04 91.44) (end 62.23 87.63) (width 0.5) (layer "F.Cu") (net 30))
 (segment (start 52.07 88.9) (end 53.34 87.63) (width 0.5) (layer "F.Cu") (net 30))
 (segment (start 66.04 91.44) (end 66.755 91.44) (width 0.5) (layer "F.Cu") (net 30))
 (segment (start 73.66 93.98) (end 68.58 88.9) (width 0.5) (layer "F.Cu") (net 16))
 (segment (start 85.09 91.44) (end 82.55 93.98) (width 0.5) (layer "F.Cu") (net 16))
 (segment (start 85.09 90.17) (end 85.09 91.44) (width 0.5) (layer "F.Cu") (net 16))
 (segment (start 68.58 88.9) (end 68.58 87.63) (width 0.5) (layer "F.Cu") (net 16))
 (segment (start 82.55 93.98) (end 73.66 93.98) (width 0.5) (layer "F.Cu") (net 16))
 (via (at 85.09 90.17) (size 1.5) (drill 0.1) (layers "F.Cu" "B.Cu") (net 16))
 (segment (start 64.215 86.36) (end 52.07 86.36) (width 0.5) (layer "F.Cu") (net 17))
 (segment (start 52.07 86.36) (end 49.53 88.9) (width 0.5) (layer "F.Cu") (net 17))
 (segment (start 65.485 87.63) (end 64.215 86.36) (width 0.5) (layer "F.Cu") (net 17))
 (segment (start 66.755 87.63) (end 65.485 87.63) (width 0.5) (layer "F.Cu") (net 17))
 (segment (start 82.55 91.44) (end 81.28 92.71) (width 0.5) (layer "F.Cu") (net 32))
 (segment (start 81.28 92.71) (end 74.93 92.71) (width 0.5) (layer "F.Cu") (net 32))
 (segment (start 82.55 90.17) (end 82.55 91.44) (width 0.5) (layer "F.Cu") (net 32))
 (segment (start 69.85 85.09) (end 68.58 83.82) (width 0.5) (layer "F.Cu") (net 32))
 (segment (start 69.85 87.63) (end 69.85 85.09) (width 0.5) (layer "F.Cu") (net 32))
 (segment (start 74.93 92.71) (end 69.85 87.63) (width 0.5) (layer "F.Cu") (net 32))
 (via (at 82.55 90.17) (size 1.5) (drill 0.1) (layers "F.Cu" "B.Cu") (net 32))
 (segment (start 50.8 85.09) (end 46.99 88.9) (width 0.5) (layer "F.Cu") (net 33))
 (segment (start 66.755 83.82) (end 65.485 83.82) (width 0.5) (layer "F.Cu") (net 33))
 (segment (start 64.215 85.09) (end 50.8 85.09) (width 0.5) (layer "F.Cu") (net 33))
 (segment (start 65.485 83.82) (end 64.215 85.09) (width 0.5) (layer "F.Cu") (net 33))
 (segment (start 80.01 90.17) (end 78.74 91.44) (width 0.5) (layer "F.Cu") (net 24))
 (segment (start 71.12 86.36) (end 71.12 82.55) (width 0.5) (layer "F.Cu") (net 24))
 (segment (start 76.2 91.44) (end 71.12 86.36) (width 0.5) (layer "F.Cu") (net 24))
 (segment (start 71.12 82.55) (end 68.58 80.01) (width 0.5) (layer "F.Cu") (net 24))
 (segment (start 78.74 91.44) (end 76.2 91.44) (width 0.5) (layer "F.Cu") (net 24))
 (via (at 80.01 90.17) (size 1.5) (drill 0.1) (layers "F.Cu" "B.Cu") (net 24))
 (segment (start 49.53 83.82) (end 44.45 88.9) (width 0.5) (layer "F.Cu") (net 25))
 (segment (start 63.5 83.82) (end 49.53 83.82) (width 0.5) (layer "F.Cu") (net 25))
 (segment (start 66.755 80.01) (end 66.755 80.565) (width 0.5) (layer "F.Cu") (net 25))
 (segment (start 66.755 80.565) (end 63.5 83.82) (width 0.5) (layer "F.Cu") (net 25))
 (segment (start 74.93 87.63) (end 72.39 85.09) (width 0.5) (layer "F.Cu") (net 27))
 (segment (start 72.39 80.01) (end 68.58 76.2) (width 0.5) (layer "F.Cu") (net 27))
 (segment (start 78.74 87.63) (end 74.93 87.63) (width 0.5) (layer "F.Cu") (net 27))
 (segment (start 68.92 75.86) (end 68.58 76.2) (width 0.5) (layer "F.Cu") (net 27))
 (segment (start 72.39 85.09) (end 72.39 80.01) (width 0.5) (layer "F.Cu") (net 27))
 (via (at 78.74 87.63) (size 1.5) (drill 0.1) (layers "F.Cu" "B.Cu") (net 27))
 (segment (start 63.5 76.2) (end 63.5 80.01) (width 0.5) (layer "F.Cu") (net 31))
 (segment (start 66.755 72.39) (end 66.755 72.945) (width 0.5) (layer "F.Cu") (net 31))
 (segment (start 63.5 80.01) (end 62.23 81.28) (width 0.5) (layer "F.Cu") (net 31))
 (segment (start 46.99 81.28) (end 39.37 88.9) (width 0.5) (layer "F.Cu") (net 31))
 (segment (start 62.23 81.28) (end 46.99 81.28) (width 0.5) (layer "F.Cu") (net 31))
 (segment (start 66.755 72.945) (end 63.5 76.2) (width 0.5) (layer "F.Cu") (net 31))
 (segment (start 54.61 43.18) (end 57.15 43.18) (width 0.5) (layer "F.Cu") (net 34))
 (segment (start 57.15 45.72) (end 54.61 45.72) (width 0.5) (layer "F.Cu") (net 35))
 (segment (start 54.61 48.26) (end 57.15 48.26) (width 0.5) (layer "F.Cu") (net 36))
 (segment (start 57.15 50.8) (end 54.61 50.8) (width 0.5) (layer "F.Cu") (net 37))
 (segment (start 54.61 53.34) (end 57.15 53.34) (width 0.5) (layer "F.Cu") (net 38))
 (segment (start 57.15 55.88) (end 54.61 55.88) (width 0.5) (layer "F.Cu") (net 39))
 (segment (start 54.61 58.42) (end 57.15 58.42) (width 0.5) (layer "F.Cu") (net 40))
 (segment (start 54.61 60.96) (end 57.15 60.96) (width 0.5) (layer "F.Cu") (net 41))
 (segment (start 57.15 63.5) (end 54.61 63.5) (width 0.5) (layer "F.Cu") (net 42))
 (segment (start 54.61 66.04) (end 57.15 66.04) (width 0.5) (layer "F.Cu") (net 43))
 (segment (start 57.15 68.58) (end 54.61 68.58) (width 0.5) (layer "F.Cu") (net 44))
 (segment (start 57.15 73.66) (end 54.61 73.66) (width 0.5) (layer "F.Cu") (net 45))
 (segment (start 54.61 76.2) (end 57.15 76.2) (width 0.5) (layer "F.Cu") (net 46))
 (segment (start 57.15 78.74) (end 54.61 78.74) (width 0.5) (layer "F.Cu") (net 47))
 (segment (start 36.83 43.18) (end 39.37 43.18) (width 0.5) (layer "F.Cu") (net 1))
 (segment (start 39.37 45.72) (end 36.83 45.72) (width 0.5) (layer "F.Cu") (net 2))
 (segment (start 36.83 48.26) (end 39.37 48.26) (width 0.5) (layer "F.Cu") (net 3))
 (segment (start 39.37 50.8) (end 36.83 50.8) (width 0.5) (layer "F.Cu") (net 4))
 (segment (start 36.83 53.34) (end 39.37 53.34) (width 0.5) (layer "F.Cu") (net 5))
 (segment (start 39.37 55.88) (end 36.83 55.88) (width 0.5) (layer "F.Cu") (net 6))
 (segment (start 36.83 58.42) (end 39.37 58.42) (width 0.5) (layer "F.Cu") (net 7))
 (segment (start 36.83 60.96) (end 39.37 60.96) (width 0.5) (layer "F.Cu") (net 8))
 (segment (start 39.37 63.5) (end 36.83 63.5) (width 0.5) (layer "F.Cu") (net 9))
 (segment (start 36.83 66.04) (end 39.37 66.04) (width 0.5) (layer "F.Cu") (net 10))
 (segment (start 41.91 88.9) (end 39.37 91.44) (width 0.5) (layer "F.Cu") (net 11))
 (segment (start 34.29 69.85) (end 35.56 68.58) (width 0.5) (layer "F.Cu") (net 11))
 (segment (start 48.26 82.55) (end 41.91 88.9) (width 0.5) (layer "F.Cu") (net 11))
 (segment (start 64.77 77.47) (end 64.77 80.645) (width 0.5) (layer "F.Cu") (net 11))
 (segment (start 36.195 91.44) (end 34.29 89.535) (width 0.5) (layer "F.Cu") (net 11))
 (segment (start 66.755 76.2) (end 66.04 76.2) (width 0.5) (layer "F.Cu") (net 11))
 (segment (start 35.56 68.58) (end 36.83 68.58) (width 0.5) (layer "F.Cu") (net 11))
 (segment (start 62.865 82.55) (end 48.26 82.55) (width 0.5) (layer "F.Cu") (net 11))
 (segment (start 39.37 68.58) (end 36.83 68.58) (width 0.5) (layer "F.Cu") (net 11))
 (segment (start 34.29 89.535) (end 34.29 69.85) (width 0.5) (layer "F.Cu") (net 11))
 (segment (start 39.37 91.44) (end 36.195 91.44) (width 0.5) (layer "F.Cu") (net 11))
 (segment (start 66.04 76.2) (end 64.77 77.47) (width 0.5) (layer "F.Cu") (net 11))
 (segment (start 64.77 80.645) (end 62.865 82.55) (width 0.5) (layer "F.Cu") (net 11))
 (segment (start 39.37 73.66) (end 36.83 73.66) (width 0.5) (layer "F.Cu") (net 13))
 (segment (start 36.83 76.2) (end 39.37 76.2) (width 0.5) (layer "F.Cu") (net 14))
 (segment (start 39.37 78.74) (end 36.83 78.74) (width 0.5) (layer "F.Cu") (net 15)))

